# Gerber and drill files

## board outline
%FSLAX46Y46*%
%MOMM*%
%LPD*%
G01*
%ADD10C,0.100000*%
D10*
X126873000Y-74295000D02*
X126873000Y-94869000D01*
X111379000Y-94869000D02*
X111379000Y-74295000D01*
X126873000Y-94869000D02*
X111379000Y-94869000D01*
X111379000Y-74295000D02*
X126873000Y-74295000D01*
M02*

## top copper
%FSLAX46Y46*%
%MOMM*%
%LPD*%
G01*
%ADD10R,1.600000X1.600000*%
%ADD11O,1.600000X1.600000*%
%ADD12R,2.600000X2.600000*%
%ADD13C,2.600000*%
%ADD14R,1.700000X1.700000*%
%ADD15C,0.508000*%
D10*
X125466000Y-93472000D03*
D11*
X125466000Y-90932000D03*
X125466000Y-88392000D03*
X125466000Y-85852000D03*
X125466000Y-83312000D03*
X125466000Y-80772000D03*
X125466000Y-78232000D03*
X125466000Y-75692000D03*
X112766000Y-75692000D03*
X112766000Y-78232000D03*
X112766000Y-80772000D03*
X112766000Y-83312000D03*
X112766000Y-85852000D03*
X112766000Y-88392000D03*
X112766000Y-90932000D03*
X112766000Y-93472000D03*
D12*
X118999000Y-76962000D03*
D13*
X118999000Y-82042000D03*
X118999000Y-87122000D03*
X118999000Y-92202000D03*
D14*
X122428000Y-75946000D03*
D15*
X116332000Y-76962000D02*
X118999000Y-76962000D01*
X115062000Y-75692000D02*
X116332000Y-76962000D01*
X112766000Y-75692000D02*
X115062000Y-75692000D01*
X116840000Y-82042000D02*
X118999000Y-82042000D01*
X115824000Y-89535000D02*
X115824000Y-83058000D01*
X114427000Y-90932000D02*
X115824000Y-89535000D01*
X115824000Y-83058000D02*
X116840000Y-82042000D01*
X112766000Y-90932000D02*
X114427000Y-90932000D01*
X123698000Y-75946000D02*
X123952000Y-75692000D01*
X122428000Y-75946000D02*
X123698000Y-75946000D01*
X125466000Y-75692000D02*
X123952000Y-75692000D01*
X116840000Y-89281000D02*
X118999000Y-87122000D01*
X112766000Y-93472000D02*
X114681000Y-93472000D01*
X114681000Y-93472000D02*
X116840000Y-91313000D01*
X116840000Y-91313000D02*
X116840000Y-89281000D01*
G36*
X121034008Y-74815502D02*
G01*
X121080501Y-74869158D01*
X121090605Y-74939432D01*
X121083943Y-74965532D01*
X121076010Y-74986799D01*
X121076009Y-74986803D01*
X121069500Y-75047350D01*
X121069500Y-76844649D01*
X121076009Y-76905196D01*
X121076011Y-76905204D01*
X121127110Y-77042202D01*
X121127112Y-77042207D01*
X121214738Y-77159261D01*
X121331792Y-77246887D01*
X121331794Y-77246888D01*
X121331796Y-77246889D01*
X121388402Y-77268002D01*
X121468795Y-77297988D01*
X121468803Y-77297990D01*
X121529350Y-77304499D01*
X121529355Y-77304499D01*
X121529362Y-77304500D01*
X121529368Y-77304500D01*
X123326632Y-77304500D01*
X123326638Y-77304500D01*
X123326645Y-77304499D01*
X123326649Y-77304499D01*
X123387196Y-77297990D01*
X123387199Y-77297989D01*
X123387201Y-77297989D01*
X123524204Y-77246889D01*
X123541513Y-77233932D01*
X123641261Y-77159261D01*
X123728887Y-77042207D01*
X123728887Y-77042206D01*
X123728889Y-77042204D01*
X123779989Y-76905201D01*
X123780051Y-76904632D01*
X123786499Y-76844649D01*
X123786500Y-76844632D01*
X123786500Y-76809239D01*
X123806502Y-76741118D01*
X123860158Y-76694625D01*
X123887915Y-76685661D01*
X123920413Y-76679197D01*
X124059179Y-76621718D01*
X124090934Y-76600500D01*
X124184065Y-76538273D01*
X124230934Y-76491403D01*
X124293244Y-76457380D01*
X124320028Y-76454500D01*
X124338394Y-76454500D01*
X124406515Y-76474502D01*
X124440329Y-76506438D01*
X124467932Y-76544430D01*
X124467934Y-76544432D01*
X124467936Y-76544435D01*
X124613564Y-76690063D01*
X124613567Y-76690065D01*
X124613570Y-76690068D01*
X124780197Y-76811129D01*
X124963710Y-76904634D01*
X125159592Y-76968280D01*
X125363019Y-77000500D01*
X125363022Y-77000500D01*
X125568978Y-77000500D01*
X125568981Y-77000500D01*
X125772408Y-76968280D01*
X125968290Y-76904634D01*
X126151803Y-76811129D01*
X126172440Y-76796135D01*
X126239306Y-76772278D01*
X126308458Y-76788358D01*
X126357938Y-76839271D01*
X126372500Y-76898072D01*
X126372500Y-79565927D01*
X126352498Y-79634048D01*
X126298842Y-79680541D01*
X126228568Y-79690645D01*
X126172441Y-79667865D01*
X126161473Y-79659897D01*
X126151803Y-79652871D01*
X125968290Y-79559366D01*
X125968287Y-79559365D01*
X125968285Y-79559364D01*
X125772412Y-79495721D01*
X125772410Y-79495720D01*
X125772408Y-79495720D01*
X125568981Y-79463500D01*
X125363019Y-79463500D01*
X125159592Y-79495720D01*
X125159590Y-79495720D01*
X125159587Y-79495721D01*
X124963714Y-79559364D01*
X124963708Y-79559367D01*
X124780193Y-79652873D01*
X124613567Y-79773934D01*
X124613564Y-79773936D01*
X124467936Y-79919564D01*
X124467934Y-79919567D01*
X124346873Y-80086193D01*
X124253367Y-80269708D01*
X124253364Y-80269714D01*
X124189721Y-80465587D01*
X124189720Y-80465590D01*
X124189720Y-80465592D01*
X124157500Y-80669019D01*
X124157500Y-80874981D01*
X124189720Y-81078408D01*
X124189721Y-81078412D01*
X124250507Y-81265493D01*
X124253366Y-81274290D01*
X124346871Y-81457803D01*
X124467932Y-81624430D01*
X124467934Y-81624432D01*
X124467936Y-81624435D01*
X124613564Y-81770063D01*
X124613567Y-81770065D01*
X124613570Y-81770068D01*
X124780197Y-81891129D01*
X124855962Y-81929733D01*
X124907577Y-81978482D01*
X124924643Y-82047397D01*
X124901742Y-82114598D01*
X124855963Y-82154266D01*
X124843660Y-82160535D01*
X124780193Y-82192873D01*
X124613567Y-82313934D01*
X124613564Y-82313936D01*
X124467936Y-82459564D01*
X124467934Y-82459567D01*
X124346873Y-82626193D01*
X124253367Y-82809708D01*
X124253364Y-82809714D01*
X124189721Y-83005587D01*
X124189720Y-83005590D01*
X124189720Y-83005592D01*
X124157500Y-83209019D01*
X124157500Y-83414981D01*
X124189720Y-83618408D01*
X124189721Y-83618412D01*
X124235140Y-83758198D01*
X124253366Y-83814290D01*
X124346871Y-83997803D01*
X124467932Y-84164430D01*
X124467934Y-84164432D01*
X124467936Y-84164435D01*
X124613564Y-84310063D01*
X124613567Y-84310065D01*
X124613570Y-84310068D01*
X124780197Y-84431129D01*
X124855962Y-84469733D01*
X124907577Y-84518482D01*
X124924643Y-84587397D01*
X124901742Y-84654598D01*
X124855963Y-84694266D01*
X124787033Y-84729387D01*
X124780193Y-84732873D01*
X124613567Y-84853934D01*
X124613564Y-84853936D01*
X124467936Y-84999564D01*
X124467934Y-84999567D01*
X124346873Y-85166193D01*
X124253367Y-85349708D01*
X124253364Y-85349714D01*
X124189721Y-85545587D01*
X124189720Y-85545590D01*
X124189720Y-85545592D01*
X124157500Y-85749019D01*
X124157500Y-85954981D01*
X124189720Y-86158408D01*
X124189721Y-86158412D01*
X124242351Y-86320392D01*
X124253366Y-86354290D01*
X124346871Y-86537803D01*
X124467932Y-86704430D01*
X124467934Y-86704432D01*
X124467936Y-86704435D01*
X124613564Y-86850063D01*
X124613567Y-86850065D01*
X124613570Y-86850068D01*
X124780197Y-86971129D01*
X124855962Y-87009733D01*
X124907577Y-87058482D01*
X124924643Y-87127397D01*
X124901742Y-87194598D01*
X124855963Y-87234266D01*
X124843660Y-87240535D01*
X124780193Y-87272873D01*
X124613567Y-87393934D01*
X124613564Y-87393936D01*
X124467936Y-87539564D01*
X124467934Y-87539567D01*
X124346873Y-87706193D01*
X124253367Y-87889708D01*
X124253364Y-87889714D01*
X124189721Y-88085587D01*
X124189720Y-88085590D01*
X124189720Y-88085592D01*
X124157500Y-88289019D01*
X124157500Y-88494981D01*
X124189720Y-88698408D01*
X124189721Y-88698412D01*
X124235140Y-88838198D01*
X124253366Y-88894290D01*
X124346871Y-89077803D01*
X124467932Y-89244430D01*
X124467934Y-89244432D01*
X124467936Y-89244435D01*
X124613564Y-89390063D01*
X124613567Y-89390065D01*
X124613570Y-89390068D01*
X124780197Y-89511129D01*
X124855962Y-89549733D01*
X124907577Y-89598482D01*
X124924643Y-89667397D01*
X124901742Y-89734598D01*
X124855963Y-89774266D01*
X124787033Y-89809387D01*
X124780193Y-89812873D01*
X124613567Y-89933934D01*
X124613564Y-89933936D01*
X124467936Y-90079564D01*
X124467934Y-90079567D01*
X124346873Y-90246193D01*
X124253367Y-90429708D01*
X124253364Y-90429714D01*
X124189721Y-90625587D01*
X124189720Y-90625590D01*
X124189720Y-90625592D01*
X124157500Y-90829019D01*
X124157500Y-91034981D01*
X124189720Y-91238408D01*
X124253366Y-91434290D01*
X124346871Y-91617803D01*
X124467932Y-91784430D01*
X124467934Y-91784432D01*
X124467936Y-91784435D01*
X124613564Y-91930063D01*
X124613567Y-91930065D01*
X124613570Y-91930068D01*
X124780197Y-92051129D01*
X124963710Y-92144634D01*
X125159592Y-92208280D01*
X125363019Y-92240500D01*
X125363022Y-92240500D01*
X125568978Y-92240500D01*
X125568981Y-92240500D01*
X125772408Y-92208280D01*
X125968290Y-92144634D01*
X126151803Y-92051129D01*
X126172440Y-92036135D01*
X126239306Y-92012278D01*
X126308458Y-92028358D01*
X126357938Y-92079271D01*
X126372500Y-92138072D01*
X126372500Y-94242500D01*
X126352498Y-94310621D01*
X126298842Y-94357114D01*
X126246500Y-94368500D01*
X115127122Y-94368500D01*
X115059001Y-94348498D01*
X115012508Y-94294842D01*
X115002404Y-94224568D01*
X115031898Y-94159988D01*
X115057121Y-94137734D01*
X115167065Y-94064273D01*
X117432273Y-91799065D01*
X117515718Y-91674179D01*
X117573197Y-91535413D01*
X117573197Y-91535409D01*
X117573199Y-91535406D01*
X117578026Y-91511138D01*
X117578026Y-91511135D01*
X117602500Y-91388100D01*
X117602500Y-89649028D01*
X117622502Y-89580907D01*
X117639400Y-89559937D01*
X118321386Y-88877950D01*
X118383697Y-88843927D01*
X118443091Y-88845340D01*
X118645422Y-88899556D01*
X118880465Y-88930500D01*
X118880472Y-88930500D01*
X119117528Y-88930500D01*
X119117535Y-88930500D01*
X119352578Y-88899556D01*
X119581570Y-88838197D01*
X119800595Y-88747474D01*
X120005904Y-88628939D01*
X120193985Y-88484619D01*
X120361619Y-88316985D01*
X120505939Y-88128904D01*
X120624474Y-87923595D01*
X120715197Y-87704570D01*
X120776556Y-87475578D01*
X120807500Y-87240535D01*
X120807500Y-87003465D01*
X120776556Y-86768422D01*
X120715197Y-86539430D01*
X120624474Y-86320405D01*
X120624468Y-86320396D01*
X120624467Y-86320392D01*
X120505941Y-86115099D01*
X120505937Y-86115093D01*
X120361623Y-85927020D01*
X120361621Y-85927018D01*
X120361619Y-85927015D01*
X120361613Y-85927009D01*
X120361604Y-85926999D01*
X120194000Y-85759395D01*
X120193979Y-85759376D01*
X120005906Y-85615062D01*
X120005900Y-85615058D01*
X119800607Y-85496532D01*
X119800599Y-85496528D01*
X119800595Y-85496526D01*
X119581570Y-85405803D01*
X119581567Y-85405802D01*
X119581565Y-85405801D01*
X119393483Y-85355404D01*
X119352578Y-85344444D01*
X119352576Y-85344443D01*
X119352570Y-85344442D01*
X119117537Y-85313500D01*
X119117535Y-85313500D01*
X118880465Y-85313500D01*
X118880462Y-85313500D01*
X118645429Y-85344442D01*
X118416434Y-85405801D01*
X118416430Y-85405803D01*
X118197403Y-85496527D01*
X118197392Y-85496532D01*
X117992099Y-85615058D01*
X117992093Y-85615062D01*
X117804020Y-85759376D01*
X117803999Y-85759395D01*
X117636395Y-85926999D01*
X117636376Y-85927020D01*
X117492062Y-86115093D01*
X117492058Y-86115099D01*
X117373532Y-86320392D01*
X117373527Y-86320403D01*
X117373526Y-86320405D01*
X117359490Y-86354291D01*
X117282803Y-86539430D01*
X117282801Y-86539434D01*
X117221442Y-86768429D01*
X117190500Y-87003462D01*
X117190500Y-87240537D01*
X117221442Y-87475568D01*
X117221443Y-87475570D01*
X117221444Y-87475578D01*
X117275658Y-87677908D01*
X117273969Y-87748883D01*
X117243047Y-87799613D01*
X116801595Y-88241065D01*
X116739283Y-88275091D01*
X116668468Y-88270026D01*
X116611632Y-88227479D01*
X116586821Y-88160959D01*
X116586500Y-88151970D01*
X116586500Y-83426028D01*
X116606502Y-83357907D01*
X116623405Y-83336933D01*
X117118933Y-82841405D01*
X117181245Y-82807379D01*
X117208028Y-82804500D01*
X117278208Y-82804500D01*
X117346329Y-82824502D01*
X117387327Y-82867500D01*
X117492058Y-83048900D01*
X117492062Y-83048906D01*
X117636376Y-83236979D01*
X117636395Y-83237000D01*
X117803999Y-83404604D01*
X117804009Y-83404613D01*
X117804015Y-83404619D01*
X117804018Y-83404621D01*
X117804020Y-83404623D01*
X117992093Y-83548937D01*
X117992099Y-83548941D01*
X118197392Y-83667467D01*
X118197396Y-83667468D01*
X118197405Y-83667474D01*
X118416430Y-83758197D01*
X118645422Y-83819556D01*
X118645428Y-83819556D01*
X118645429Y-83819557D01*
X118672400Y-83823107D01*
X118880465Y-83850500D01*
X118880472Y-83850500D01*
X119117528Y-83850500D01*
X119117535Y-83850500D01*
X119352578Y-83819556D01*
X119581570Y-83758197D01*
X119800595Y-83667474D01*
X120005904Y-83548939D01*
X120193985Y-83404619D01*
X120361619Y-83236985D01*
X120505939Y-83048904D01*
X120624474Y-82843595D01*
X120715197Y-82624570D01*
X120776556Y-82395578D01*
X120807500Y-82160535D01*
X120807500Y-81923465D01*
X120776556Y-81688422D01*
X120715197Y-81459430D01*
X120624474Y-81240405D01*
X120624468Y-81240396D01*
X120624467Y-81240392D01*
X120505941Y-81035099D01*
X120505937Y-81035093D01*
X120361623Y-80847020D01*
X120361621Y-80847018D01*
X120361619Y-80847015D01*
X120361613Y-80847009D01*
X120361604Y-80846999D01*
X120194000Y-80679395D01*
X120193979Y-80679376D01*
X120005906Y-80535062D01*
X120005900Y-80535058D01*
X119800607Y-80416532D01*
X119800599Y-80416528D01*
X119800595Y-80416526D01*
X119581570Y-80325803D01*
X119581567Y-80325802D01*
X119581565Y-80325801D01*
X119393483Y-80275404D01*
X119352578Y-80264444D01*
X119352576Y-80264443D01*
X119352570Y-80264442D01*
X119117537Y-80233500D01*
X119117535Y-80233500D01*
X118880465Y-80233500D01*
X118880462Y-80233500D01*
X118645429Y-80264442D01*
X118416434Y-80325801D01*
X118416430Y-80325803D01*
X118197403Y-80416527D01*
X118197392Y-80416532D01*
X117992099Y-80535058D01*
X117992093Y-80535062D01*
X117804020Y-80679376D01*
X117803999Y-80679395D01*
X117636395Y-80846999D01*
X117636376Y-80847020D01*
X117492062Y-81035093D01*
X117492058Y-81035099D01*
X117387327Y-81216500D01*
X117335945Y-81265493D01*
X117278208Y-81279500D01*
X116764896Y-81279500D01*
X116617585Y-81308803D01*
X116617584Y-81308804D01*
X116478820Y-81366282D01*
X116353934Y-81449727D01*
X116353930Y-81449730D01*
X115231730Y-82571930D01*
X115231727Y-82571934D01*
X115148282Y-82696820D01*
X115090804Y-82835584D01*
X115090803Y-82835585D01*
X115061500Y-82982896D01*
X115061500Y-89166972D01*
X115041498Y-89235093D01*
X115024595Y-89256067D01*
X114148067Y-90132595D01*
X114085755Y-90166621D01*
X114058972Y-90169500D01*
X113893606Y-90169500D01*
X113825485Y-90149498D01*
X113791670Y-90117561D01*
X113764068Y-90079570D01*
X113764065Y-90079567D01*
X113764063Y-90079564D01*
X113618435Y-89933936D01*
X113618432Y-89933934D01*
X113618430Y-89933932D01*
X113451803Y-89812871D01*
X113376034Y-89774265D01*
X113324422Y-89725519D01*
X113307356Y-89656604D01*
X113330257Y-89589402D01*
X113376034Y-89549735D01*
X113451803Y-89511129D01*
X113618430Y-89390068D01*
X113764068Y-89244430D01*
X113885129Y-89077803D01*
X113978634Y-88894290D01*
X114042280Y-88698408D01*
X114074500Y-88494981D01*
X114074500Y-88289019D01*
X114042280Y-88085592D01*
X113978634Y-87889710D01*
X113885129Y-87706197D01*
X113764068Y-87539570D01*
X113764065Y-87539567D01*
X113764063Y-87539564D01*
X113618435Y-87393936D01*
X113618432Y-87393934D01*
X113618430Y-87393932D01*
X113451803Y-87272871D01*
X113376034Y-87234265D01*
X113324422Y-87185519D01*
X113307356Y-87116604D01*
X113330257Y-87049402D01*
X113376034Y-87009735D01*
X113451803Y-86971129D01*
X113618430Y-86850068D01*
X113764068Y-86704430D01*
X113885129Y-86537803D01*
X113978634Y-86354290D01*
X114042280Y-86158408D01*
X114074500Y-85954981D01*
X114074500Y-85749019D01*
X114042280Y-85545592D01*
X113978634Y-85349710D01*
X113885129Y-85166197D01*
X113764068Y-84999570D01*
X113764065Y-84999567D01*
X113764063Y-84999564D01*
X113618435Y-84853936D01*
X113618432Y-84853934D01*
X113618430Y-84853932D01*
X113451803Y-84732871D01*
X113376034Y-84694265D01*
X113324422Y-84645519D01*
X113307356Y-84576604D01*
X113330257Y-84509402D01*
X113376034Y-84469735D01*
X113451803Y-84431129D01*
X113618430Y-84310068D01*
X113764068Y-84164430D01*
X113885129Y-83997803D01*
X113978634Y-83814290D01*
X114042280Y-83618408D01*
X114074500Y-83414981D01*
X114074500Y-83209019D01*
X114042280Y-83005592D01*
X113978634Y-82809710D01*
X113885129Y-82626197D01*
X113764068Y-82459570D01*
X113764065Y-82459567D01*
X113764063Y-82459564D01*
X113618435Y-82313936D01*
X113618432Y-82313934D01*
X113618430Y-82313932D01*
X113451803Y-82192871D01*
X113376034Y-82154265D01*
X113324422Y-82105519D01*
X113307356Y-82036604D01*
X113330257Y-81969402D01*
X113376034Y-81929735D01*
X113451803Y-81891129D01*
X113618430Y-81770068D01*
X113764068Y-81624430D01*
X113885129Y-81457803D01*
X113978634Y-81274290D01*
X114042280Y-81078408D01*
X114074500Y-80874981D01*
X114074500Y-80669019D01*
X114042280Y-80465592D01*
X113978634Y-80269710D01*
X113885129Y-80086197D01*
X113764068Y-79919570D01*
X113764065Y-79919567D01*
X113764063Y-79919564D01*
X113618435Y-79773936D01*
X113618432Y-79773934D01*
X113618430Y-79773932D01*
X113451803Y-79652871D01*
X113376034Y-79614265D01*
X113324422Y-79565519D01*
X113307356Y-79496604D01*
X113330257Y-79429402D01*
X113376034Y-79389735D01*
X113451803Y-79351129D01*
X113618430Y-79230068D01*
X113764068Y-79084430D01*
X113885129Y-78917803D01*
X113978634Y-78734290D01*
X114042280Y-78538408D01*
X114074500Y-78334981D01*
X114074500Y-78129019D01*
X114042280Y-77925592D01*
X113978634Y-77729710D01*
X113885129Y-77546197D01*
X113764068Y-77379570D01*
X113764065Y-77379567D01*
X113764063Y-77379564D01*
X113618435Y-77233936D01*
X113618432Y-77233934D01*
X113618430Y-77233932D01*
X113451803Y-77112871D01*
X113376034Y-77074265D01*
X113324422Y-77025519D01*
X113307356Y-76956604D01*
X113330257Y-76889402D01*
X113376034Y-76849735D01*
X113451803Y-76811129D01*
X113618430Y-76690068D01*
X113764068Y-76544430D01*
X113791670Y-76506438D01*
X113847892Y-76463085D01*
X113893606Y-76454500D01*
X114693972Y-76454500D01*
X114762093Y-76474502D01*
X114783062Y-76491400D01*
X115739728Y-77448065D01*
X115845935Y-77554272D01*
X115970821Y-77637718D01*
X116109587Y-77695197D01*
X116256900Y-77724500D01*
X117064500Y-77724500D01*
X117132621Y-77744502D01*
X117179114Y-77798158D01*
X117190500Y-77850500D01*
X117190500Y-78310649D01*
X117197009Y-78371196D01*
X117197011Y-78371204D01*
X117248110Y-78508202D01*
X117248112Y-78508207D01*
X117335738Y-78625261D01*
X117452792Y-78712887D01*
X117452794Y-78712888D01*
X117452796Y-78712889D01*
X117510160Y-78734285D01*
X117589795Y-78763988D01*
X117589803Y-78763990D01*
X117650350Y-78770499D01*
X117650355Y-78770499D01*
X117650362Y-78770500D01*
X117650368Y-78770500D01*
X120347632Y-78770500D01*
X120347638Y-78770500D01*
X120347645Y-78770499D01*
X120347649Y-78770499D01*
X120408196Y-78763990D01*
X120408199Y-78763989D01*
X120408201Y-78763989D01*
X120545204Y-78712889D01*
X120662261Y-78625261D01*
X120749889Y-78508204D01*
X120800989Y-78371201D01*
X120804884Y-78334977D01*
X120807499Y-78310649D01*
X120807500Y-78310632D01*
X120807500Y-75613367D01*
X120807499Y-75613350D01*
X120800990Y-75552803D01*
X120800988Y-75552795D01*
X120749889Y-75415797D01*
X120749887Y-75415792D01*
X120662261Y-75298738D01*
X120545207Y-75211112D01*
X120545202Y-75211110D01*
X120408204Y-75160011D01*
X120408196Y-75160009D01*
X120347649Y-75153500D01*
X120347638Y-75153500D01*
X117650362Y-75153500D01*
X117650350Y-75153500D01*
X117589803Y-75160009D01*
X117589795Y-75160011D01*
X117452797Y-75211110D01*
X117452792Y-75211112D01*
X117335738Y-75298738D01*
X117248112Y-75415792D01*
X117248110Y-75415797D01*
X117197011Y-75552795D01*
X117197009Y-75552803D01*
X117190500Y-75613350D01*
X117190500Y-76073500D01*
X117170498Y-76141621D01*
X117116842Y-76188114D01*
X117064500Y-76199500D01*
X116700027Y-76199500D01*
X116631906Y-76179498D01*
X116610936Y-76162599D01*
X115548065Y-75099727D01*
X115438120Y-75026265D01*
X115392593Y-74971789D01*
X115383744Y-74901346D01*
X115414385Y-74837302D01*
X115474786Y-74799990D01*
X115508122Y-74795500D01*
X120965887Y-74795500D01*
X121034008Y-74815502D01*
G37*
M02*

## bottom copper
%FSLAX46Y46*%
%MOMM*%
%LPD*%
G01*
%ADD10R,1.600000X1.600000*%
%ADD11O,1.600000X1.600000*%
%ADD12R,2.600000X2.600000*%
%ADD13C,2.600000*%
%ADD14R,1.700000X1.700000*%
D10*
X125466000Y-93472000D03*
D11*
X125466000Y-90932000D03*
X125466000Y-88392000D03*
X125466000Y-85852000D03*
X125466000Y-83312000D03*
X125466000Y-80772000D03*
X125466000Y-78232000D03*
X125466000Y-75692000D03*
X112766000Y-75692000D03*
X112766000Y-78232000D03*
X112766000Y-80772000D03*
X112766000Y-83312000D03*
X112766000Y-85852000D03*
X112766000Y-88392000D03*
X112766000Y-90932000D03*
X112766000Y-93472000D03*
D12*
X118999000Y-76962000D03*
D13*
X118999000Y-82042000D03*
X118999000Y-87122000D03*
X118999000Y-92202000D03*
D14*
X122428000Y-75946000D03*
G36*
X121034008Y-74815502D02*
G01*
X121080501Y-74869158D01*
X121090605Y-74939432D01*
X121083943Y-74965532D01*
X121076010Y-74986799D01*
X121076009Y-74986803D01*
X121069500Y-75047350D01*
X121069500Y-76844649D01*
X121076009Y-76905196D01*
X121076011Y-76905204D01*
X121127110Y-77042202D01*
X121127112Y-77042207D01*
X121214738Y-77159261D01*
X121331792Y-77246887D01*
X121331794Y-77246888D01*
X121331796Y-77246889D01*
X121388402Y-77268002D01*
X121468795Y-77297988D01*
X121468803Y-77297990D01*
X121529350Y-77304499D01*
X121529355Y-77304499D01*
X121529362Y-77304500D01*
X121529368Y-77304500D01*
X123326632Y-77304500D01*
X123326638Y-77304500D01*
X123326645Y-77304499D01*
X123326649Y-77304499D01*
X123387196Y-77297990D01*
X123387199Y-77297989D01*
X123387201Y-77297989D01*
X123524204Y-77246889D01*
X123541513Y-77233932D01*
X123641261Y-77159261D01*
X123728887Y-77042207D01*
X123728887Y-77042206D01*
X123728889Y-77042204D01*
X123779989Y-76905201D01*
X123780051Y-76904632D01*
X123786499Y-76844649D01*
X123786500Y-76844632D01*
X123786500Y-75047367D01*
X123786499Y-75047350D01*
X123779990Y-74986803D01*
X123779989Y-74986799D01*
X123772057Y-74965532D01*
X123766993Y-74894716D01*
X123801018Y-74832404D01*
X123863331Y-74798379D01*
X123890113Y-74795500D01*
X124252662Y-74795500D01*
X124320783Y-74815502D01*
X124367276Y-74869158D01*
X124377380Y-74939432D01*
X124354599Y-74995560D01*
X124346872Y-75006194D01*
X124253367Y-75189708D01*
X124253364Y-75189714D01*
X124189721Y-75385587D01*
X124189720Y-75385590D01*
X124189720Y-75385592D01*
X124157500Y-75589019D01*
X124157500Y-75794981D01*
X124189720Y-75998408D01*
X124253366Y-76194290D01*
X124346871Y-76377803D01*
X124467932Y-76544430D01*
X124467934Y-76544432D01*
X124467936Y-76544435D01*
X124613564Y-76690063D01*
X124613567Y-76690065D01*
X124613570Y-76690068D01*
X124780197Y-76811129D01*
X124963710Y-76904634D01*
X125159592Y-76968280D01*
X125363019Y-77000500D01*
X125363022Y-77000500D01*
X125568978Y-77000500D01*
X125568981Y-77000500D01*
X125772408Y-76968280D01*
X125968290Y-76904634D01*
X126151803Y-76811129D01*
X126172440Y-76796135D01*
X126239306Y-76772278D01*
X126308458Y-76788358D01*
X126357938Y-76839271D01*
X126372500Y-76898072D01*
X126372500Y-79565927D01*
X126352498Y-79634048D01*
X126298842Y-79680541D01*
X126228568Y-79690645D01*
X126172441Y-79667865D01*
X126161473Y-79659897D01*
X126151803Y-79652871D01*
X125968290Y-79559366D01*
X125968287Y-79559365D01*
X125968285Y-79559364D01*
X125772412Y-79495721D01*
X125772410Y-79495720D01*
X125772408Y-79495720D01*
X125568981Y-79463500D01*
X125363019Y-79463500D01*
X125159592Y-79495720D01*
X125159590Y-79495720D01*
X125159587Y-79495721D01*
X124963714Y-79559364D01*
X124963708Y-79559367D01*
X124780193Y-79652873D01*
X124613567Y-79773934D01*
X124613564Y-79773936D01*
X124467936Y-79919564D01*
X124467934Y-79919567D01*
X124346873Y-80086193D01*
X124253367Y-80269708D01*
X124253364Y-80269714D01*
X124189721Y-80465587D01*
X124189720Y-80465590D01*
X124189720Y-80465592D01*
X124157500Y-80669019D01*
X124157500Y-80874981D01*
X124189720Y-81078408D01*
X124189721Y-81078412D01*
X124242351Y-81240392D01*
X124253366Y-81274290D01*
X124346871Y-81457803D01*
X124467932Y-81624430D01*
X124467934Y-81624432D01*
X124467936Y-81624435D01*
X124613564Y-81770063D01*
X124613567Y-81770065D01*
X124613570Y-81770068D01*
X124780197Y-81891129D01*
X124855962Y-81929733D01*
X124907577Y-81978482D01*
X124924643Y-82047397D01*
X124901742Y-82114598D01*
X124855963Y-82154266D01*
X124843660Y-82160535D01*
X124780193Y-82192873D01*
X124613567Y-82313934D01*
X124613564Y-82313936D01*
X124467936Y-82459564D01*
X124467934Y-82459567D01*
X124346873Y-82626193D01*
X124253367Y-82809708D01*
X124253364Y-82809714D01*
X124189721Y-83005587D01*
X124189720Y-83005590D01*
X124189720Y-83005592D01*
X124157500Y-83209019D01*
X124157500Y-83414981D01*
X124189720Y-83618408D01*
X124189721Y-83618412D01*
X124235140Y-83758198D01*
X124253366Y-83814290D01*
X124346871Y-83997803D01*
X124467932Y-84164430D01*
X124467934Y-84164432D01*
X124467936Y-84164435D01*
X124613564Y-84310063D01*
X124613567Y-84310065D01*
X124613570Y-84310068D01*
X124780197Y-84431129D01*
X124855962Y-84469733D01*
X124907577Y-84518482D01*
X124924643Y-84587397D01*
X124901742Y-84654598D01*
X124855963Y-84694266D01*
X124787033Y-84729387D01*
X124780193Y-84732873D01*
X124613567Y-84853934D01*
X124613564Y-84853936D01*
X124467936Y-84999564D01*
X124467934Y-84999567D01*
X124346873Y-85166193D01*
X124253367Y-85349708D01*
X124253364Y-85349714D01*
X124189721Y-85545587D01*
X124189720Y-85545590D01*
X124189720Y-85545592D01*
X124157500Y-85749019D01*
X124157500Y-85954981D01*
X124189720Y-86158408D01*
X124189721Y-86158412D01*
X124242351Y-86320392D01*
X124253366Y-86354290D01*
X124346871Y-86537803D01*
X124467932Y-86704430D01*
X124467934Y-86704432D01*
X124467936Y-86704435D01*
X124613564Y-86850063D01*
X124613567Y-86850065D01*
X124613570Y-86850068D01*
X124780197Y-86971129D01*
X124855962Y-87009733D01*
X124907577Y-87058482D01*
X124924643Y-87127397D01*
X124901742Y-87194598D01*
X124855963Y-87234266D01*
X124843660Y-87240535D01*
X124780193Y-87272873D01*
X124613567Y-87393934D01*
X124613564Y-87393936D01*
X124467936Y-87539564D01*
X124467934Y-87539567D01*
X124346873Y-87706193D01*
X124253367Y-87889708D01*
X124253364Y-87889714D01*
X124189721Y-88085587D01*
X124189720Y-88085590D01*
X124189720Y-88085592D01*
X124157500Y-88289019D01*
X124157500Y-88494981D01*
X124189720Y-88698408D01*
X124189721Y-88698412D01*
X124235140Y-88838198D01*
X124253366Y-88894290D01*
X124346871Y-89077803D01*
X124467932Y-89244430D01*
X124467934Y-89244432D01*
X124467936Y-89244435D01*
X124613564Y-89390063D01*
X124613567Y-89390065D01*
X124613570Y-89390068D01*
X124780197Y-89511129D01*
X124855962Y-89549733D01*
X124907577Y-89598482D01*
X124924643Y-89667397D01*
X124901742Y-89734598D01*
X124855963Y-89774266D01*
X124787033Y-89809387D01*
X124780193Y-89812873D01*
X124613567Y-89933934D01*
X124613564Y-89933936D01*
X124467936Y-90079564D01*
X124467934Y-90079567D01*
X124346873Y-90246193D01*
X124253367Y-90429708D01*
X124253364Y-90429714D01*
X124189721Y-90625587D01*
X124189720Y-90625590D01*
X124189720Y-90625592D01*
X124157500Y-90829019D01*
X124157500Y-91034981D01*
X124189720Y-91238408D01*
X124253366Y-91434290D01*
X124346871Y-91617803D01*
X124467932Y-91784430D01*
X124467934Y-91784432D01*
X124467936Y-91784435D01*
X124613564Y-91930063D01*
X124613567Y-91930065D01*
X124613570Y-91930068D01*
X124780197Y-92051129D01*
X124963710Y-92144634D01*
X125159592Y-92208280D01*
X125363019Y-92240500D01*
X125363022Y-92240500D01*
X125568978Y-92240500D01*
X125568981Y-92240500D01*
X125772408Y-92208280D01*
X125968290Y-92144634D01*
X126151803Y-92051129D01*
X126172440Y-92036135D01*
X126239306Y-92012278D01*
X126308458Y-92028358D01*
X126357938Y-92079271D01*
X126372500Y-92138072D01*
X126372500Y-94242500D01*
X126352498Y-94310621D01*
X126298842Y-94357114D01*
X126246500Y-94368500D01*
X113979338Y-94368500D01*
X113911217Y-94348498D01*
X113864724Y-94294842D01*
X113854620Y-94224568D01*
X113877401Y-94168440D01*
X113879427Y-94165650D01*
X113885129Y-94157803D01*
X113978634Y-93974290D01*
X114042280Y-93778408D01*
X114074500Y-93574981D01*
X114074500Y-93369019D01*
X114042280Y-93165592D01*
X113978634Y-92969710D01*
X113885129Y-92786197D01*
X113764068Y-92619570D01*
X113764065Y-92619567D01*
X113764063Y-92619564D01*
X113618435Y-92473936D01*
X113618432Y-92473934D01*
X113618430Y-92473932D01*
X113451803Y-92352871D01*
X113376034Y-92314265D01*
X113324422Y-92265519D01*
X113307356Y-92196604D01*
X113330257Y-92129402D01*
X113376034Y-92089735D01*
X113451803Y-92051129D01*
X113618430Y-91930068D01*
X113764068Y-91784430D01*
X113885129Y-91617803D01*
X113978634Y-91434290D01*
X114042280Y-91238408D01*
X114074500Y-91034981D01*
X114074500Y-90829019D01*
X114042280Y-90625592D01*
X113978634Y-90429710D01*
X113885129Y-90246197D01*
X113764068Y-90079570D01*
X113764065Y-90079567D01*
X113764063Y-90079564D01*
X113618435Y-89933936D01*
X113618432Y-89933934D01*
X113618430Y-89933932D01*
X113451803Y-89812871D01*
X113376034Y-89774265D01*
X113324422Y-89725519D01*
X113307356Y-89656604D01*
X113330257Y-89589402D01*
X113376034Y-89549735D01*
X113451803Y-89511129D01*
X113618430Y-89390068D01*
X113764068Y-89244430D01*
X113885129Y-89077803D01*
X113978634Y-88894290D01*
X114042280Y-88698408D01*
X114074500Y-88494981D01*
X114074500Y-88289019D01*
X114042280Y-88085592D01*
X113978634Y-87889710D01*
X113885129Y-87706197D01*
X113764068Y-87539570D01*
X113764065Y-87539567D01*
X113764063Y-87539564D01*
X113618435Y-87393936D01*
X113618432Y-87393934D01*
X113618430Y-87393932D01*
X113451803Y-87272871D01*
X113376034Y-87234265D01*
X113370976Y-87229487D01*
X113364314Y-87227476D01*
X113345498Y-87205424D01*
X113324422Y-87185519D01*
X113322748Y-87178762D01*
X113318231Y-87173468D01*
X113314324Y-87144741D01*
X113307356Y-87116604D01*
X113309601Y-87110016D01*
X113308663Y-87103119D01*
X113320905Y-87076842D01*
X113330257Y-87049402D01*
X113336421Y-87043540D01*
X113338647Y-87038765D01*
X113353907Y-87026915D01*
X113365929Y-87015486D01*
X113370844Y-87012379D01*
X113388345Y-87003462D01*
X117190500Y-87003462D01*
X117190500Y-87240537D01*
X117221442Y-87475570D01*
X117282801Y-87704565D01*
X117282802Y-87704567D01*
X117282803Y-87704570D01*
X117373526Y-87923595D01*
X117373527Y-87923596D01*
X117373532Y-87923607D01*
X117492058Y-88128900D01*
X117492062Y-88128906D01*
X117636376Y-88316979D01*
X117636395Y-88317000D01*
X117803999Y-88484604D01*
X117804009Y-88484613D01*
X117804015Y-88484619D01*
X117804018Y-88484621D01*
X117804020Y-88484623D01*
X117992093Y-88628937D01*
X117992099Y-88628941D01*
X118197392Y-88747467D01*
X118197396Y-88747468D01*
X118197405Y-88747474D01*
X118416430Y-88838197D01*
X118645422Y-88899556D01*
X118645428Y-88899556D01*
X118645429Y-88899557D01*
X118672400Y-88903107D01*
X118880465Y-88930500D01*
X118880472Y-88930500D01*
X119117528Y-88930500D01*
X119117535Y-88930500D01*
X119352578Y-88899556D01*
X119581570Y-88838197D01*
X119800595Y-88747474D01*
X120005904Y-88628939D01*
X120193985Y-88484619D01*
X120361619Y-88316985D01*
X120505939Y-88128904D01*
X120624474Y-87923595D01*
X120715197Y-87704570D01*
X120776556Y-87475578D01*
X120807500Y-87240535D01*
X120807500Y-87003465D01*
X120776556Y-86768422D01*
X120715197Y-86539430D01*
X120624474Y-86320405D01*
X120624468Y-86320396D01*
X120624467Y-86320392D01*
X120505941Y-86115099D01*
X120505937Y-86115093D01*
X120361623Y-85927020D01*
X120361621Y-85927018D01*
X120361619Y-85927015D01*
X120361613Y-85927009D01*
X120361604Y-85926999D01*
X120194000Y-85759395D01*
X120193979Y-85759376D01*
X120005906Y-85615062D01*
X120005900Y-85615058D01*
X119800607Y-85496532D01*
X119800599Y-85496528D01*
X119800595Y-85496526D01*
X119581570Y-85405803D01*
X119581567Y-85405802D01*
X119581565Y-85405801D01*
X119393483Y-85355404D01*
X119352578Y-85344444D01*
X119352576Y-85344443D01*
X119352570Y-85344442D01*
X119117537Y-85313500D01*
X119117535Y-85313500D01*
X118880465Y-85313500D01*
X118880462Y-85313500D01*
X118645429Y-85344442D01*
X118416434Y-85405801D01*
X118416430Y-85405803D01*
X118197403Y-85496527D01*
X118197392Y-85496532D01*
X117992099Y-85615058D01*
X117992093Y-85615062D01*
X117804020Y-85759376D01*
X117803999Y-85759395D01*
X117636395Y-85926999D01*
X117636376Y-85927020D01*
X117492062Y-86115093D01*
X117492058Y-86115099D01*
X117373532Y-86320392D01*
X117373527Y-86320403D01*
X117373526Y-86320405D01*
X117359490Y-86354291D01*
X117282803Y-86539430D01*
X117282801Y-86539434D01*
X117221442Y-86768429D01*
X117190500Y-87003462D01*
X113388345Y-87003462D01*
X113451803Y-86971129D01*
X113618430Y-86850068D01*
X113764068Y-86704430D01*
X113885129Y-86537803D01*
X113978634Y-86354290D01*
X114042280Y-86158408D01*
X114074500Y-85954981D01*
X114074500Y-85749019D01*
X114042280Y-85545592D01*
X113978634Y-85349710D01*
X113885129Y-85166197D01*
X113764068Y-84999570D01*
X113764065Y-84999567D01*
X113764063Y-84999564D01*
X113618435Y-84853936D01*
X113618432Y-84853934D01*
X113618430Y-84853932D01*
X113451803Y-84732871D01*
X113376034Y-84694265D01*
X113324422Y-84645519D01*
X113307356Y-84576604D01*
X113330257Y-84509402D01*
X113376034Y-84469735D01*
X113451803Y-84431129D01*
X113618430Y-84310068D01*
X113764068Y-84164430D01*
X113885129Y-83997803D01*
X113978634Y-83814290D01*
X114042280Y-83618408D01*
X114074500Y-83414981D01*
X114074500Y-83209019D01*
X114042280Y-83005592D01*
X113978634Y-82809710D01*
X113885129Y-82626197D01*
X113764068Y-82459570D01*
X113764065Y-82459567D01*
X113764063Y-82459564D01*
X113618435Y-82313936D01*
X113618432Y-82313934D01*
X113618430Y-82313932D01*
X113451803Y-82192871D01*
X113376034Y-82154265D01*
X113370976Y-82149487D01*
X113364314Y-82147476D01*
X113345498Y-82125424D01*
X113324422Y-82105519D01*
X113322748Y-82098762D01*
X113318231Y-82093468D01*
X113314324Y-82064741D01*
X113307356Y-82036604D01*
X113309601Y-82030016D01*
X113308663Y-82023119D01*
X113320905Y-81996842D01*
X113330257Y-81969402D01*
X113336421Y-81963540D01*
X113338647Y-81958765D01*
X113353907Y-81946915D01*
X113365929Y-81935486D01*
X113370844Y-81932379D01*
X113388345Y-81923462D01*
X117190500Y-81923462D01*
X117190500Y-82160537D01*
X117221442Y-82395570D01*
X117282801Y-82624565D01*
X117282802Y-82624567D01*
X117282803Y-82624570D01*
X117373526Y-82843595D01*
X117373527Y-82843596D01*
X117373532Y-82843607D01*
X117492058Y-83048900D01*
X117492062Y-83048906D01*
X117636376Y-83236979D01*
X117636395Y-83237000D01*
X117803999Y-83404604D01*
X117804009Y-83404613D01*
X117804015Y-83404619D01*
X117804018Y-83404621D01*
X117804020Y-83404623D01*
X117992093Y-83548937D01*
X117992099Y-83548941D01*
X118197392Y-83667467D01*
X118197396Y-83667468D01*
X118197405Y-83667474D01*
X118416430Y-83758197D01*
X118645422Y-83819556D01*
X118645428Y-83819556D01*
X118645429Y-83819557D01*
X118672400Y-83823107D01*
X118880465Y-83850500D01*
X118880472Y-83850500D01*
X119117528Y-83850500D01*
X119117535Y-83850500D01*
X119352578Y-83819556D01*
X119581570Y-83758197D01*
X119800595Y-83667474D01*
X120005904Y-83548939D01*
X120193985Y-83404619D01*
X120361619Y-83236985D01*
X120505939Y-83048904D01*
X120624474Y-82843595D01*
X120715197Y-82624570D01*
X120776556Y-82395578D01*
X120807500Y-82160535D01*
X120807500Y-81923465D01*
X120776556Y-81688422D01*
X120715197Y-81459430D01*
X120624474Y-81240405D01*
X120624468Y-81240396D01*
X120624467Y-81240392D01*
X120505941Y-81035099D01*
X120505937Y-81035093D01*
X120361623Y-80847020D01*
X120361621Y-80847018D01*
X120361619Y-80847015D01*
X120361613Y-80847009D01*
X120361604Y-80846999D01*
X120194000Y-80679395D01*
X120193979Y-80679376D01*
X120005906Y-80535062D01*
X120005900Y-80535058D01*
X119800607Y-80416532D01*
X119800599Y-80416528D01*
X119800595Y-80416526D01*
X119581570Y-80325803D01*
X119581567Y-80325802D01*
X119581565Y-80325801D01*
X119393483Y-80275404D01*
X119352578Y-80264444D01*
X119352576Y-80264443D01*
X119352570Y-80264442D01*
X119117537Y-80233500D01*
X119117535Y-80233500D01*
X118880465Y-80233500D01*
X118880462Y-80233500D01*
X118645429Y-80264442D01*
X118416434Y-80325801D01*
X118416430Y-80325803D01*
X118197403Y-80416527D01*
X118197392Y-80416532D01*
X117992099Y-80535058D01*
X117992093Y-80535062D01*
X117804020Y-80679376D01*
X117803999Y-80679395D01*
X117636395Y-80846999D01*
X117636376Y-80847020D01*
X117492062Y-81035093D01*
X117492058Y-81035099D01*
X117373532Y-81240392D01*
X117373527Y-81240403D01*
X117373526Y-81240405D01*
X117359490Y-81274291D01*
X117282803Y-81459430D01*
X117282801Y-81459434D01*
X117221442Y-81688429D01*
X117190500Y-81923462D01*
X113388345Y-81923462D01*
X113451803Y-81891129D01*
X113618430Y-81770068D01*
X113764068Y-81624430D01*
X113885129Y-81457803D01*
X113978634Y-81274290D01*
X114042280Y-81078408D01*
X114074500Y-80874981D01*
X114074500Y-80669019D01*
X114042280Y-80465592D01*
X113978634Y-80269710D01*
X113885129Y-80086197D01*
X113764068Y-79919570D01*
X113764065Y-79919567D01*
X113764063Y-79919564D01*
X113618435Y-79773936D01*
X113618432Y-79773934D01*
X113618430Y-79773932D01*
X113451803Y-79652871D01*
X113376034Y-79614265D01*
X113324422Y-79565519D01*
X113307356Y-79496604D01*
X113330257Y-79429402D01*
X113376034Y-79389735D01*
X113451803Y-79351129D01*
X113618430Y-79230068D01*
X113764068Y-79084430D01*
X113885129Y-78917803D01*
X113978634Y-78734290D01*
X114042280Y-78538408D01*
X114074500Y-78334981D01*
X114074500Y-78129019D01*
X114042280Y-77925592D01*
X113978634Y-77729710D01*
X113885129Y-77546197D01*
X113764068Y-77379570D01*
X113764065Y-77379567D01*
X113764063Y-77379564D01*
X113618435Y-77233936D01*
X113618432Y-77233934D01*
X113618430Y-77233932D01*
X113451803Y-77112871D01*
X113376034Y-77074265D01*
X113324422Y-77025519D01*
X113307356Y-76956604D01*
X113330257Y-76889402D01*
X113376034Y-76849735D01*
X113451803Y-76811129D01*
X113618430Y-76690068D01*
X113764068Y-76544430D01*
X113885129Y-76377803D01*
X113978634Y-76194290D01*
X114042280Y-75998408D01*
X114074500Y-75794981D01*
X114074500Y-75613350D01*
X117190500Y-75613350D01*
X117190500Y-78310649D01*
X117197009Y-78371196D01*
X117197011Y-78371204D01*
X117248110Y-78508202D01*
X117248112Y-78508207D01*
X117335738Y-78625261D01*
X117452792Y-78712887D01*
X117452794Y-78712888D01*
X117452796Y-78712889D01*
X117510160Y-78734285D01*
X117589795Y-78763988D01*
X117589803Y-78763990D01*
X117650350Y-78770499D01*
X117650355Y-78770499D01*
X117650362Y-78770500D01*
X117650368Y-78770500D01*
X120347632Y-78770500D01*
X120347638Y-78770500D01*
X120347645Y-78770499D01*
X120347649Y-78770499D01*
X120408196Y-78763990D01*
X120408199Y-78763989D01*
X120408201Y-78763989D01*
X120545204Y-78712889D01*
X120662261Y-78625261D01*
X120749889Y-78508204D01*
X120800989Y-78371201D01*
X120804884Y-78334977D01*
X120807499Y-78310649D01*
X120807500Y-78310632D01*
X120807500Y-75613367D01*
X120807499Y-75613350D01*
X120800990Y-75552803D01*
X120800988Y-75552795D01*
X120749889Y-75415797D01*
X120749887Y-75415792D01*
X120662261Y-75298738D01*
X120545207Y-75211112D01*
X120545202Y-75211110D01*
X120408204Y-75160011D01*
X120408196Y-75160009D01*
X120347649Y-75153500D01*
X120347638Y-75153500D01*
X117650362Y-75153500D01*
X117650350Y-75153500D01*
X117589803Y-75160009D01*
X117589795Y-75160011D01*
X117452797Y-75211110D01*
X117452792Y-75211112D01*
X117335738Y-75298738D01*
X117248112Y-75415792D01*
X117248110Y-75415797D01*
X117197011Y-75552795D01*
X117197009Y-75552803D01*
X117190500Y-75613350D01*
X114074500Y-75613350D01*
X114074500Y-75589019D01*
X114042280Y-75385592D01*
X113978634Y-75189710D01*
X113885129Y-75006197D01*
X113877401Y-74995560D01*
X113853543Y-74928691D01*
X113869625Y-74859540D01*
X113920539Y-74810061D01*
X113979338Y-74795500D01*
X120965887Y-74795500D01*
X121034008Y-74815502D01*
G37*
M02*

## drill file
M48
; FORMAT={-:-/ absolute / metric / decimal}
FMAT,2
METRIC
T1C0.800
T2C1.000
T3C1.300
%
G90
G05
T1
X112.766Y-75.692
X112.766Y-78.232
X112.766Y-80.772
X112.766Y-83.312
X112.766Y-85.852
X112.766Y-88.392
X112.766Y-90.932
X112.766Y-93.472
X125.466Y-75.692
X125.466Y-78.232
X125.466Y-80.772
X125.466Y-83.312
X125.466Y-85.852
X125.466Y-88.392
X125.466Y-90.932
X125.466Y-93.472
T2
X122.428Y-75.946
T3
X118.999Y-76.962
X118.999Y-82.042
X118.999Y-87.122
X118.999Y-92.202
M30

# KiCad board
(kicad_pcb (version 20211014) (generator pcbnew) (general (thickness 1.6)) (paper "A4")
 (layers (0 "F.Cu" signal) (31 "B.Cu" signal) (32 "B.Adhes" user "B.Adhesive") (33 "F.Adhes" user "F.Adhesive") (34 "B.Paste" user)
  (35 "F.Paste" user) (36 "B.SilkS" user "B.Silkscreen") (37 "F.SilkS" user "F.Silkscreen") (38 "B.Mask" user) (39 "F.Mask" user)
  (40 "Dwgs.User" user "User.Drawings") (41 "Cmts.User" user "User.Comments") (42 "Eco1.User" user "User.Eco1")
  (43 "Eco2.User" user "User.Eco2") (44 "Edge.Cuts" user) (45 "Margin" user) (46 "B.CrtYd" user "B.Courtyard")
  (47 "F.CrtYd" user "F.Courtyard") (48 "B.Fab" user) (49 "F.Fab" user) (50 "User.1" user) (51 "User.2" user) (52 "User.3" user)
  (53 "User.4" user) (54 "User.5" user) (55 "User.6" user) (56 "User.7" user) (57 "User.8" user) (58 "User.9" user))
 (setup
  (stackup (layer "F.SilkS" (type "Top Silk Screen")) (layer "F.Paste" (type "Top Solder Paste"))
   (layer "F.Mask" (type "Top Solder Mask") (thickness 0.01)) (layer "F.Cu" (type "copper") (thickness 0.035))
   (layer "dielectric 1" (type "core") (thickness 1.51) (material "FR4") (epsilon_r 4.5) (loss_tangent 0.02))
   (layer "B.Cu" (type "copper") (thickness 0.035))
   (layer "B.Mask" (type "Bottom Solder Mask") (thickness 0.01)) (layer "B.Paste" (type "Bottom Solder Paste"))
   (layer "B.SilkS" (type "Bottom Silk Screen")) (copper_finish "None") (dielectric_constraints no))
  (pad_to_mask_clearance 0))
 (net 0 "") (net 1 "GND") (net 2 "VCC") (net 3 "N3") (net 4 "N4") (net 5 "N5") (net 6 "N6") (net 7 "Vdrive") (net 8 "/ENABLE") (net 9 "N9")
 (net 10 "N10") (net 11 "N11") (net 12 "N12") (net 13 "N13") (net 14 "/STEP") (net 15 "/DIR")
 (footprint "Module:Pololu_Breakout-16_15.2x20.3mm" (layer "F.Cu") (at 125.466 93.472 180)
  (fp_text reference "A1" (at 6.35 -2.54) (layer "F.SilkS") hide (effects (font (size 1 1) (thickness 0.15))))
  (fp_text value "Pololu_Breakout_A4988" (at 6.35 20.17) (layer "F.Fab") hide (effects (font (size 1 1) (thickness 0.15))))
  (pad "1" thru_hole rect locked (at 0 0 180) (size 1.6 1.6) (drill 0.8) (layers *.Cu *.Mask) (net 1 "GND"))
  (pad "2" thru_hole oval locked (at 0 2.54 180) (size 1.6 1.6) (drill 0.8) (layers *.Cu *.Mask) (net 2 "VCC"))
  (pad "3" thru_hole oval locked (at 0 5.08 180) (size 1.6 1.6) (drill 0.8) (layers *.Cu *.Mask) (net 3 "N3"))
  (pad "4" thru_hole oval locked (at 0 7.62 180) (size 1.6 1.6) (drill 0.8) (layers *.Cu *.Mask) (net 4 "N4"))
  (pad "5" thru_hole oval locked (at 0 10.16 180) (size 1.6 1.6) (drill 0.8) (layers *.Cu *.Mask) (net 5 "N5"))
  (pad "6" thru_hole oval locked (at 0 12.7 180) (size 1.6 1.6) (drill 0.8) (layers *.Cu *.Mask) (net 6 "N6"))
  (pad "7" thru_hole oval locked (at 0 15.24 180) (size 1.6 1.6) (drill 0.8) (layers *.Cu *.Mask) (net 1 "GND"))
  (pad "8" thru_hole oval locked (at 0 17.78 180) (size 1.6 1.6) (drill 0.8) (layers *.Cu *.Mask) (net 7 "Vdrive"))
  (pad "9" thru_hole oval locked (at 12.7 17.78 180) (size 1.6 1.6) (drill 0.8) (layers *.Cu *.Mask) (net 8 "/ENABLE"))
  (pad "10" thru_hole oval locked (at 12.7 15.24 180) (size 1.6 1.6) (drill 0.8) (layers *.Cu *.Mask) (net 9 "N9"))
  (pad "11" thru_hole oval locked (at 12.7 12.7 180) (size 1.6 1.6) (drill 0.8) (layers *.Cu *.Mask) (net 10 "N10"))
  (pad "12" thru_hole oval locked (at 12.7 10.16 180) (size 1.6 1.6) (drill 0.8) (layers *.Cu *.Mask) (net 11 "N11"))
  (pad "13" thru_hole oval locked (at 12.7 7.62 180) (size 1.6 1.6) (drill 0.8) (layers *.Cu *.Mask) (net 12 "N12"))
  (pad "14" thru_hole oval locked (at 12.7 5.08 180) (size 1.6 1.6) (drill 0.8) (layers *.Cu *.Mask) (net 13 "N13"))
  (pad "15" thru_hole oval locked (at 12.7 2.54 180) (size 1.6 1.6) (drill 0.8) (layers *.Cu *.Mask) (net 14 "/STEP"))
  (pad "16" thru_hole oval locked (at 12.7 0 180) (size 1.6 1.6) (drill 0.8) (layers *.Cu *.Mask) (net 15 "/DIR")))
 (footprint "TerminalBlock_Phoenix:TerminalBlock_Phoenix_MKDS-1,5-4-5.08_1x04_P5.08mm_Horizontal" (layer "F.Cu") (at 118.999 76.962 -90)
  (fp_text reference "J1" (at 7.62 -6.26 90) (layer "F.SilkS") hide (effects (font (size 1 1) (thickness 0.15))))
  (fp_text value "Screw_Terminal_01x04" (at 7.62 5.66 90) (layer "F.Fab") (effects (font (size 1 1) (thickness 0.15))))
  (pad "1" thru_hole rect locked (at 0 0 270) (size 2.6 2.6) (drill 1.3) (layers *.Cu *.Mask) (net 8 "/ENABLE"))
  (pad "2" thru_hole circle locked (at 5.08 0 270) (size 2.6 2.6) (drill 1.3) (layers *.Cu *.Mask) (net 14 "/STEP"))
  (pad "3" thru_hole circle locked (at 10.16 0 270) (size 2.6 2.6) (drill 1.3) (layers *.Cu *.Mask) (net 15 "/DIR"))
  (pad "4" thru_hole circle locked (at 15.24 0 270) (size 2.6 2.6) (drill 1.3) (layers *.Cu *.Mask) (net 1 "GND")))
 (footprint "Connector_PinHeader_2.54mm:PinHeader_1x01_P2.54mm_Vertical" (layer "F.Cu") (at 122.428 75.946)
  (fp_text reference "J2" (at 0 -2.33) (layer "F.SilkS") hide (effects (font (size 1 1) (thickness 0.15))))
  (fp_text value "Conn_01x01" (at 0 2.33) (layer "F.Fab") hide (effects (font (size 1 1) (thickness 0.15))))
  (pad "1" thru_hole rect locked (at 0 0) (size 1.7 1.7) (drill 1) (layers *.Cu *.Mask) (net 7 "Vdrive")))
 (gr_line (start 126.873 74.295) (end 126.873 94.869) (layer "Edge.Cuts") (width 0.1))
 (gr_line (start 111.379 94.869) (end 111.379 74.295) (layer "Edge.Cuts") (width 0.1))
 (gr_line (start 126.873 94.869) (end 111.379 94.869) (layer "Edge.Cuts") (width 0.1))
 (gr_line (start 111.379 74.295) (end 126.873 74.295) (layer "Edge.Cuts") (width 0.1))
 (segment (start 116.332 76.962) (end 118.999 76.962) (width 0.508) (layer "F.Cu") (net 8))
 (segment (start 115.062 75.692) (end 116.332 76.962) (width 0.508) (layer "F.Cu") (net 8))
 (segment (start 112.766 75.692) (end 115.062 75.692) (width 0.508) (layer "F.Cu") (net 8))
 (segment (start 116.84 82.042) (end 118.999 82.042) (width 0.508) (layer "F.Cu") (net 14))
 (segment (start 115.824 89.535) (end 115.824 83.058) (width 0.508) (layer "F.Cu") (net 14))
 (segment (start 114.427 90.932) (end 115.824 89.535) (width 0.508) (layer "F.Cu") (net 14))
 (segment (start 115.824 83.058) (end 116.84 82.042) (width 0.508) (layer "F.Cu") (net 14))
 (segment (start 112.766 90.932) (end 114.427 90.932) (width 0.508) (layer "F.Cu") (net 14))
 (segment (start 123.698 75.946) (end 123.952 75.692) (width 0.508) (layer "F.Cu") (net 7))
 (segment (start 122.428 75.946) (end 123.698 75.946) (width 0.508) (layer "F.Cu") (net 7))
 (segment (start 125.466 75.692) (end 123.952 75.692) (width 0.508) (layer "F.Cu") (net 7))
 (segment (start 116.84 89.281) (end 118.999 87.122) (width 0.508) (layer "F.Cu") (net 15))
 (segment (start 112.766 93.472) (end 114.681 93.472) (width 0.508) (layer "F.Cu") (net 15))
 (segment (start 114.681 93.472) (end 116.84 91.313) (width 0.508) (layer "F.Cu") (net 15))
 (segment (start 116.84 91.313) (end 116.84 89.281) (width 0.508) (layer "F.Cu") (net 15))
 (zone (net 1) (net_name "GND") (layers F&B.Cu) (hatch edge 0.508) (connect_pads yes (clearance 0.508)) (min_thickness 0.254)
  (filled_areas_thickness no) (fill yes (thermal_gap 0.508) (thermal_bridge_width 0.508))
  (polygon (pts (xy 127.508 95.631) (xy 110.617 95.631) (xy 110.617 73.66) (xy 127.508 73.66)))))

